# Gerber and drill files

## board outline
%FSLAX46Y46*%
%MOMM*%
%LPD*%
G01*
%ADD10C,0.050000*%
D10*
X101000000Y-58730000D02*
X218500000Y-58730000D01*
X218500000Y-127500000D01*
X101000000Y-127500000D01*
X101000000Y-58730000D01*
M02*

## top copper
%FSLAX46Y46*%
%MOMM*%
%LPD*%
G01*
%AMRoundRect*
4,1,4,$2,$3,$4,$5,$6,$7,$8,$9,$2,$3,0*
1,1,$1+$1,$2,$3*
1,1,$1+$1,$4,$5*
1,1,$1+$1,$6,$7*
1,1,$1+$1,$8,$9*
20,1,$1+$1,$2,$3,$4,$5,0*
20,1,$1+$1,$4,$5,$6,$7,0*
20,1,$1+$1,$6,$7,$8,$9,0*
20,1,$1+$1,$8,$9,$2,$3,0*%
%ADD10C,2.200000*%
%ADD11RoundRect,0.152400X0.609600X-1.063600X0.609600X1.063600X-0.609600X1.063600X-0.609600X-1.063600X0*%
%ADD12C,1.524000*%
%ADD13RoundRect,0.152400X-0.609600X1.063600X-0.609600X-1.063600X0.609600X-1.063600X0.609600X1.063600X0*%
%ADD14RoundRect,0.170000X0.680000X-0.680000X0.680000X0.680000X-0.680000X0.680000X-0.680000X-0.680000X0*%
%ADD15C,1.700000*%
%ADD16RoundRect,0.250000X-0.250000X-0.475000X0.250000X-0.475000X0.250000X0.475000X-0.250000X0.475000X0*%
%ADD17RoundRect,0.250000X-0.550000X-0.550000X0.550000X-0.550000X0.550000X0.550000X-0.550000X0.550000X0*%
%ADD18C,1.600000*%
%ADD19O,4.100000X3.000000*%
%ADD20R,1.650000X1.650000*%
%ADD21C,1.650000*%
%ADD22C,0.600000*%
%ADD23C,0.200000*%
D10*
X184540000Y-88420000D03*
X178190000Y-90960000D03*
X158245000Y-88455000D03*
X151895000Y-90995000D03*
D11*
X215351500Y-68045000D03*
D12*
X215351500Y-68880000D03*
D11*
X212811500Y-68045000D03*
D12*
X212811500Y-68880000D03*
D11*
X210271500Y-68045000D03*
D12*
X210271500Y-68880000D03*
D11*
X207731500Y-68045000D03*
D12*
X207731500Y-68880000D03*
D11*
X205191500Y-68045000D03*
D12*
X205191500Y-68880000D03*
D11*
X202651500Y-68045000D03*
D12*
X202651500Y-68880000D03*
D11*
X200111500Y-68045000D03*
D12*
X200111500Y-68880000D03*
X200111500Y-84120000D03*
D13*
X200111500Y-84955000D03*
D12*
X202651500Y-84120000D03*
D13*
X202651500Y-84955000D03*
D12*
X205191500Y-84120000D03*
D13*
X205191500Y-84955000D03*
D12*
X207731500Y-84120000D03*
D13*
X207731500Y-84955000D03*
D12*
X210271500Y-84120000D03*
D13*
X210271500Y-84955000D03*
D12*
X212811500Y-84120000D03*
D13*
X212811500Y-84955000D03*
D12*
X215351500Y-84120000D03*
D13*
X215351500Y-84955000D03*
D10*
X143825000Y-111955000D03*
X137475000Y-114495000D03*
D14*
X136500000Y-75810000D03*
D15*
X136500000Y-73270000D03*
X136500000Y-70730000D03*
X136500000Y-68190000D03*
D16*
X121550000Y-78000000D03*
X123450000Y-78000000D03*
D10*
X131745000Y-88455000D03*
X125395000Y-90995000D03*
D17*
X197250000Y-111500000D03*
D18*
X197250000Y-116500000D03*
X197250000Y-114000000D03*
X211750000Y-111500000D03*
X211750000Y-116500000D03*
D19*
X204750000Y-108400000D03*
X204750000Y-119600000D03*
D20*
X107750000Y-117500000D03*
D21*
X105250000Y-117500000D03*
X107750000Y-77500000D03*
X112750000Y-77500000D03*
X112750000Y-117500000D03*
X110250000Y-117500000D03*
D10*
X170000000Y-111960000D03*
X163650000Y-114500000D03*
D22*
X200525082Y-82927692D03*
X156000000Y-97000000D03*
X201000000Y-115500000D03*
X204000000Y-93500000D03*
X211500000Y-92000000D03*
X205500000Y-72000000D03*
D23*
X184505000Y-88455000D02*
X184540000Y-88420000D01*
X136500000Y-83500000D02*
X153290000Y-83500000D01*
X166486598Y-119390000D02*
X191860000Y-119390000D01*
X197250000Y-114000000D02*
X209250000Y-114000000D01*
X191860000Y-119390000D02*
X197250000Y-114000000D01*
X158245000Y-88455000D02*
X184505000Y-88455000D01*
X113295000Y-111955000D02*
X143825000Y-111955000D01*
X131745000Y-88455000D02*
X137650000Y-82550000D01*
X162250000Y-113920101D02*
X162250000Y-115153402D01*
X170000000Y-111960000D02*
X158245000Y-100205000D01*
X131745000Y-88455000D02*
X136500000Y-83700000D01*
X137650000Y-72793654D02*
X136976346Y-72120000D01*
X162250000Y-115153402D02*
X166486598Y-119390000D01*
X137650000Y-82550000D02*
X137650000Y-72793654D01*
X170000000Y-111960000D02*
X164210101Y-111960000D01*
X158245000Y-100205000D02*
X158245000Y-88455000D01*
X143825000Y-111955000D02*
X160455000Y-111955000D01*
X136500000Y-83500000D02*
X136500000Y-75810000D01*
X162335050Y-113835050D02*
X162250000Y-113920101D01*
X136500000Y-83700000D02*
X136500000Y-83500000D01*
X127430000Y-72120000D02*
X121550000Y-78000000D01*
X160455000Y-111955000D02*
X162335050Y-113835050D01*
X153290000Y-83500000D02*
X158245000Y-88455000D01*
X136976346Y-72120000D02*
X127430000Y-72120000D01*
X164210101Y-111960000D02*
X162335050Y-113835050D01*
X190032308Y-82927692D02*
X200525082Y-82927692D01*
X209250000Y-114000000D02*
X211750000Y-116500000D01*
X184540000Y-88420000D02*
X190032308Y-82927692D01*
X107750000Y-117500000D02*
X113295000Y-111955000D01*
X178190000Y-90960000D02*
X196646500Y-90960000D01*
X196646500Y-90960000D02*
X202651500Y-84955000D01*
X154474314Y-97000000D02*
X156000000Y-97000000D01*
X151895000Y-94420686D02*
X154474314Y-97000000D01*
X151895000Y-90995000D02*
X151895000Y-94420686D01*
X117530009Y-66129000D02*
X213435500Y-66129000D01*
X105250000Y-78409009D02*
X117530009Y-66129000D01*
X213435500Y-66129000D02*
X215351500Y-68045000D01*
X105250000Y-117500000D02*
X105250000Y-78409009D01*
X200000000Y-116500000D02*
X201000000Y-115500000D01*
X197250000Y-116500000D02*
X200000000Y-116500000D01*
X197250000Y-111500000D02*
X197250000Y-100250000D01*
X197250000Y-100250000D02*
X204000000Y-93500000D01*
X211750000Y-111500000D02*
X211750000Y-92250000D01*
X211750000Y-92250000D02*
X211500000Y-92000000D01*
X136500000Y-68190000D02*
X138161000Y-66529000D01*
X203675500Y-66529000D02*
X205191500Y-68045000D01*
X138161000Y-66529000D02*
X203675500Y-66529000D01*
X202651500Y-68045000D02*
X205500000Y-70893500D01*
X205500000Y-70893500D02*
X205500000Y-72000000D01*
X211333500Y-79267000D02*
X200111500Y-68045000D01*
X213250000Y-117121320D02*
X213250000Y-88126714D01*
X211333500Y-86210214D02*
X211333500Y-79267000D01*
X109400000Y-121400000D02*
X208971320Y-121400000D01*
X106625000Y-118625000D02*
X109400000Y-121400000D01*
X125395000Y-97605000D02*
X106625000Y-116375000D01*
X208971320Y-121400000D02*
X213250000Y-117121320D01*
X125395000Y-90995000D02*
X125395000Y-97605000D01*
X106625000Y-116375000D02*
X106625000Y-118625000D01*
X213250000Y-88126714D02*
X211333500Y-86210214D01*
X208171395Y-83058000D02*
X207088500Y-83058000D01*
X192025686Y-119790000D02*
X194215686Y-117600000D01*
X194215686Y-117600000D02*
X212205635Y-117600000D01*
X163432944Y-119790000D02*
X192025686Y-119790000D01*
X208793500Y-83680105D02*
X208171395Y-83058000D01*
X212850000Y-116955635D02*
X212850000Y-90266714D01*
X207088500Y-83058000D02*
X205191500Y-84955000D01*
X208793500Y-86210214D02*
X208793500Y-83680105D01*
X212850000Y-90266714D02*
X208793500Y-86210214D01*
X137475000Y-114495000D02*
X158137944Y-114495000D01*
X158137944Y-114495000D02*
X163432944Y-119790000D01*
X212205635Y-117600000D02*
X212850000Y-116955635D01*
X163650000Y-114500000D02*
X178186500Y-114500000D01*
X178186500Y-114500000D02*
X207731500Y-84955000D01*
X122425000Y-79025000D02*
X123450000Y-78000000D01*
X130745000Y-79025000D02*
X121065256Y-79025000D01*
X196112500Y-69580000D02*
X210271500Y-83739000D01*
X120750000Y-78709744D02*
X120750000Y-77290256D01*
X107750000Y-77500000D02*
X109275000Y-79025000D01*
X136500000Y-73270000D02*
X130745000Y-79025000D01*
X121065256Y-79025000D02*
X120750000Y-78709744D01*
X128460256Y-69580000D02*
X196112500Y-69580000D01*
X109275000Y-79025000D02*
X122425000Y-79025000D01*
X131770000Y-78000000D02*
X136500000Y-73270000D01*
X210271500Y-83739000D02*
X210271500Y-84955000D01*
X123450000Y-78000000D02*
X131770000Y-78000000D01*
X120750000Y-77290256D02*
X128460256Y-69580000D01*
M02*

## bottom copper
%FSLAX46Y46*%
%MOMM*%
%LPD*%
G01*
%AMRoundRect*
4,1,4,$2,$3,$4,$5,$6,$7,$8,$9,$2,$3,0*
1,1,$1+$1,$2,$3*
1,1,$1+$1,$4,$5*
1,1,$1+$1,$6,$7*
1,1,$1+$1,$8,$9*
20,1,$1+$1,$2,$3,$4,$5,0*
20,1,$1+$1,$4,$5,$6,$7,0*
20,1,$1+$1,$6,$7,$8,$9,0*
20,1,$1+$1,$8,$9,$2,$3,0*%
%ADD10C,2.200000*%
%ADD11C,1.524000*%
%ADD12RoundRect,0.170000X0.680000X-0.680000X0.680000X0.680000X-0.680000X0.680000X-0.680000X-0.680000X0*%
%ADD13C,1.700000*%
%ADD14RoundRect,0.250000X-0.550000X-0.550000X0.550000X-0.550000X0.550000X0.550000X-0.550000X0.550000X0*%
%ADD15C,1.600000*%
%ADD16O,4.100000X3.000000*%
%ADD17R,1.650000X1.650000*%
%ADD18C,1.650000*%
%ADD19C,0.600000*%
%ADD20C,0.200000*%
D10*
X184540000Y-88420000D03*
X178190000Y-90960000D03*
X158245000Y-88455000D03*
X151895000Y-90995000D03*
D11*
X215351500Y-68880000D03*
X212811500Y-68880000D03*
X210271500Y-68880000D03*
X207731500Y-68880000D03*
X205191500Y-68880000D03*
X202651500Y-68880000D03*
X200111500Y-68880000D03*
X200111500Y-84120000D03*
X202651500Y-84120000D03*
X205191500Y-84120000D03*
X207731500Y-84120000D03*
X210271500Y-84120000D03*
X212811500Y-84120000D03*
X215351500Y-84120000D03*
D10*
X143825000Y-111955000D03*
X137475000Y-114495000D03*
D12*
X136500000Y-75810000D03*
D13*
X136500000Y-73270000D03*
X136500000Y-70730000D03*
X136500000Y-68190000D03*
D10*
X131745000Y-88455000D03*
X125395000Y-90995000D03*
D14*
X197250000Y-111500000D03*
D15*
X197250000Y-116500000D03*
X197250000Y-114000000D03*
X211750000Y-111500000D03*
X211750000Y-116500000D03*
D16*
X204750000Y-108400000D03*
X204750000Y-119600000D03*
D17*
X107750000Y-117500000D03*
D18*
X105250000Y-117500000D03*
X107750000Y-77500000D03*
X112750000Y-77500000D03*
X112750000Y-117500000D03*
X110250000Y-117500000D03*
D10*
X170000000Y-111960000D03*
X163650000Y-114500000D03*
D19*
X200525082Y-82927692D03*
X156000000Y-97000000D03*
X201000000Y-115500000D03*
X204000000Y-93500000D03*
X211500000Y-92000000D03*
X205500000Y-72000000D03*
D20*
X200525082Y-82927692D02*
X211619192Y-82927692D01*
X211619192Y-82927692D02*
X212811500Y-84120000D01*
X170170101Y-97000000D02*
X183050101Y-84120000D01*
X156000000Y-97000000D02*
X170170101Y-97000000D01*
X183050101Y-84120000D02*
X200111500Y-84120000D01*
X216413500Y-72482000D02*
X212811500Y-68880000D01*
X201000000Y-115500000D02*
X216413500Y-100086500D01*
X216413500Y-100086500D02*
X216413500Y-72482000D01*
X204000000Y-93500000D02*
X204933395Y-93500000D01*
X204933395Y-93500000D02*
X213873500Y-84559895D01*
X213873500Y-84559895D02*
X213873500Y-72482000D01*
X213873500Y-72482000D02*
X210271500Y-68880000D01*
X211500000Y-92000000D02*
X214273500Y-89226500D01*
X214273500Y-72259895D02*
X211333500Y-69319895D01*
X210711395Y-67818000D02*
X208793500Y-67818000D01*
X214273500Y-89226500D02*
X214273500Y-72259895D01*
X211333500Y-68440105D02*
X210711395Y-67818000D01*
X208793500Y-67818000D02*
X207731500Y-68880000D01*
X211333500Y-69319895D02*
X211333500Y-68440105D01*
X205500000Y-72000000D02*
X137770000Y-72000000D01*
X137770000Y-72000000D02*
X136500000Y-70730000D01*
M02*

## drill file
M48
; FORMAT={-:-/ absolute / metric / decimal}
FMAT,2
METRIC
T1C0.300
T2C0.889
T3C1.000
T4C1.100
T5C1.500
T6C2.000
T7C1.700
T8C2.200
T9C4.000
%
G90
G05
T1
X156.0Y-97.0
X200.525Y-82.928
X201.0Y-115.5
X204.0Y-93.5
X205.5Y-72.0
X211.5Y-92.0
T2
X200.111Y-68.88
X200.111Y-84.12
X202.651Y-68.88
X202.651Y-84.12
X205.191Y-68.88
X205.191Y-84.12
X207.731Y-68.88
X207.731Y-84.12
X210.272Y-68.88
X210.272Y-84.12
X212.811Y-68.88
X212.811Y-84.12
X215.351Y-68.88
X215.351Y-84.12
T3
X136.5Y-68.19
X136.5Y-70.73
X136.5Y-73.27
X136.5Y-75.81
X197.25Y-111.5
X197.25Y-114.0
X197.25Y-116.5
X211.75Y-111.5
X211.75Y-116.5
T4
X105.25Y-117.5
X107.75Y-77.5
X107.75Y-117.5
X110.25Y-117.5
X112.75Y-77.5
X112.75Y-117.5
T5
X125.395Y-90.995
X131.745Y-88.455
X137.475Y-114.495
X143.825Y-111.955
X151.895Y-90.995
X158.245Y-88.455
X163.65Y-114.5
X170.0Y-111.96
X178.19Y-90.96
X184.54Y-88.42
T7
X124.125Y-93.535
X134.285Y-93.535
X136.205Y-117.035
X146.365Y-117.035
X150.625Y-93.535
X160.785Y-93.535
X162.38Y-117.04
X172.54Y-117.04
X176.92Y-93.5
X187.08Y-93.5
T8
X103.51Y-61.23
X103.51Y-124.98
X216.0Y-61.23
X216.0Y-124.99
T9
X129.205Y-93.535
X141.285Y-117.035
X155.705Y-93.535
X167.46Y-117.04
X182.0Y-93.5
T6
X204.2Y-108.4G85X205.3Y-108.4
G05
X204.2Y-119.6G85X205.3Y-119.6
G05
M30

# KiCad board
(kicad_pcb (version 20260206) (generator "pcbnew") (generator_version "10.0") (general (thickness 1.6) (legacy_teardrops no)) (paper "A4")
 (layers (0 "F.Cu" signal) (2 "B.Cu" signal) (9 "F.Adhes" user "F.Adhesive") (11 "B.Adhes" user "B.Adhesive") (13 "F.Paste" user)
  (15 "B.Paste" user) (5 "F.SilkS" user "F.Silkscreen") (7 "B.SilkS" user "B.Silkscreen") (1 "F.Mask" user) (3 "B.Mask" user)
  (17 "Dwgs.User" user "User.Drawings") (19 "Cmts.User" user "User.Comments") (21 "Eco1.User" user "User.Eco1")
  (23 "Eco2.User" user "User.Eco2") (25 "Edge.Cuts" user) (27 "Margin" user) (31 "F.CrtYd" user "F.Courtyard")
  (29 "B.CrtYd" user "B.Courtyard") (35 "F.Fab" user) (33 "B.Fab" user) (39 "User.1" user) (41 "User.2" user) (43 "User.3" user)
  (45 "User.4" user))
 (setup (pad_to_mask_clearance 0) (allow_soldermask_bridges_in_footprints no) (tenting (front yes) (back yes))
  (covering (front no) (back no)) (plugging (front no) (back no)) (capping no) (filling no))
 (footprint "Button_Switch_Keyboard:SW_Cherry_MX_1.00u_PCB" (layer "F.Cu") (at 184.54 88.42)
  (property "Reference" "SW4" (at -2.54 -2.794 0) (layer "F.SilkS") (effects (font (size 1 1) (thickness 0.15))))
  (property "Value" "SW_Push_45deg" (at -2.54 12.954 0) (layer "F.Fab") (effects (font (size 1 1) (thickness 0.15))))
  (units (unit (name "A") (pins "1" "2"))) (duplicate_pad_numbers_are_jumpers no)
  (pad "" np_thru_hole circle (at -7.62 5.08) (size 1.7 1.7) (drill 1.7) (layers "*.Cu" "*.Mask"))
  (pad "" np_thru_hole circle (at -2.54 5.08) (size 4 4) (drill 4) (layers "*.Cu" "*.Mask"))
  (pad "" np_thru_hole circle (at 2.54 5.08) (size 1.7 1.7) (drill 1.7) (layers "*.Cu" "*.Mask"))
  (pad "1" thru_hole circle (at 0 0) (size 2.2 2.2) (drill 1.5) (layers "*.Cu" "*.Mask") (remove_unused_layers no) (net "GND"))
  (pad "2" thru_hole circle (at -6.35 2.54) (size 2.2 2.2) (drill 1.5) (layers "*.Cu" "*.Mask") (remove_unused_layers no) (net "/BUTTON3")))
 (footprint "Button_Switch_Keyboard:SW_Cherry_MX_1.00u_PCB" (layer "F.Cu") (at 158.245 88.455)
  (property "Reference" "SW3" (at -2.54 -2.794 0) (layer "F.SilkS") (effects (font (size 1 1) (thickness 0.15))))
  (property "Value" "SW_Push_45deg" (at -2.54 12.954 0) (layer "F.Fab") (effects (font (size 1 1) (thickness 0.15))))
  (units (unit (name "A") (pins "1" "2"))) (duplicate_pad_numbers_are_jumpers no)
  (pad "" np_thru_hole circle (at -7.62 5.08) (size 1.7 1.7) (drill 1.7) (layers "*.Cu" "*.Mask"))
  (pad "" np_thru_hole circle (at -2.54 5.08) (size 4 4) (drill 4) (layers "*.Cu" "*.Mask"))
  (pad "" np_thru_hole circle (at 2.54 5.08) (size 1.7 1.7) (drill 1.7) (layers "*.Cu" "*.Mask"))
  (pad "1" thru_hole circle (at 0 0) (size 2.2 2.2) (drill 1.5) (layers "*.Cu" "*.Mask") (remove_unused_layers no) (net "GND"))
  (pad "2" thru_hole circle (at -6.35 2.54) (size 2.2 2.2) (drill 1.5) (layers "*.Cu" "*.Mask") (remove_unused_layers no) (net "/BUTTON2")))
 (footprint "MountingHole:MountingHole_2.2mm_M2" (layer "F.Cu") (at 216 124.99)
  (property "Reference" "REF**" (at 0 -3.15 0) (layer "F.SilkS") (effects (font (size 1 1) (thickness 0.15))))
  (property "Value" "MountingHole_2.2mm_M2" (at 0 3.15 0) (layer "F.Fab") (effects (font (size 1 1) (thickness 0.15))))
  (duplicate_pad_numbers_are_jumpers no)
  (pad "" np_thru_hole circle (at 0 0) (size 2.2 2.2) (drill 2.2) (layers "*.Cu" "*.Mask")))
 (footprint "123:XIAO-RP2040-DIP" (layer "F.Cu") (at 207.7315 76.5)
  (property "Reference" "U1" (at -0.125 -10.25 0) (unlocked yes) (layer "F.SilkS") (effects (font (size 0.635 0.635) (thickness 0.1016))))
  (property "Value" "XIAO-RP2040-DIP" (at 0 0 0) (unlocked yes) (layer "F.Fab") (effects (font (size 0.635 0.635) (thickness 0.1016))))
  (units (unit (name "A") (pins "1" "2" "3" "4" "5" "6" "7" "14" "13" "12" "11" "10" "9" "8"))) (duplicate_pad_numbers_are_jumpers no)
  (pad "1" smd roundrect (at 7.62 -8.455 90) (size 2.432 1.524) (layers "F.Cu" "F.Mask") (roundrect_rratio 0.1) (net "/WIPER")
   (thermal_bridge_angle 45))
  (pad "1" thru_hole circle (at 7.62 -7.62 90) (size 1.524 1.524) (drill 0.889) (layers "*.Cu" "*.Mask") (remove_unused_layers no)
   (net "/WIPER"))
  (pad "2" smd roundrect (at 5.08 -8.455 90) (size 2.432 1.524) (layers "F.Cu" "F.Mask") (roundrect_rratio 0.1) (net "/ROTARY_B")
   (thermal_bridge_angle 45))
  (pad "2" thru_hole circle (at 5.08 -7.62 90) (size 1.524 1.524) (drill 0.889) (layers "*.Cu" "*.Mask") (remove_unused_layers no)
   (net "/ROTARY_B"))
  (pad "3" smd roundrect (at 2.54 -8.455 90) (size 2.432 1.524) (layers "F.Cu" "F.Mask") (roundrect_rratio 0.1) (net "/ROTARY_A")
   (thermal_bridge_angle 45))
  (pad "3" thru_hole circle (at 2.54 -7.62 90) (size 1.524 1.524) (drill 0.889) (layers "*.Cu" "*.Mask") (remove_unused_layers no)
   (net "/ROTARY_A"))
  (pad "4" smd roundrect (at 0 -8.455 90) (size 2.432 1.524) (layers "F.Cu" "F.Mask") (roundrect_rratio 0.1) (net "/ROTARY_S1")
   (thermal_bridge_angle 45))
  (pad "4" thru_hole circle (at 0 -7.62 90) (size 1.524 1.524) (drill 0.889) (layers "*.Cu" "*.Mask") (remove_unused_layers no)
   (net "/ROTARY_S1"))
  (pad "5" smd roundrect (at -2.54 -8.455 90) (size 2.432 1.524) (layers "F.Cu" "F.Mask") (roundrect_rratio 0.1) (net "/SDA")
   (thermal_bridge_angle 45))
  (pad "5" thru_hole circle (at -2.54 -7.62 90) (size 1.524 1.524) (drill 0.889) (layers "*.Cu" "*.Mask") (remove_unused_layers no)
   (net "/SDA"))
  (pad "6" smd roundrect (at -5.08 -8.455 90) (size 2.432 1.524) (layers "F.Cu" "F.Mask") (roundrect_rratio 0.1) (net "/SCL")
   (thermal_bridge_angle 45))
  (pad "6" thru_hole circle (at -5.08 -7.62 90) (size 1.524 1.524) (drill 0.889) (layers "*.Cu" "*.Mask") (remove_unused_layers no)
   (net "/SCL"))
  (pad "7" smd roundrect (at -7.62 -8.455 90) (size 2.432 1.524) (layers "F.Cu" "F.Mask") (roundrect_rratio 0.1) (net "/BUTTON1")
   (thermal_bridge_angle 45))
  (pad "7" thru_hole circle (at -7.62 -7.62 90) (size 1.524 1.524) (drill 0.889) (layers "*.Cu" "*.Mask") (remove_unused_layers no)
   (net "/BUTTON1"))
  (pad "8" thru_hole circle (at -7.62 7.62 270) (size 1.524 1.524) (drill 0.889) (layers "*.Cu" "*.Mask") (remove_unused_layers no)
   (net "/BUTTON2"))
  (pad "8" smd roundrect (at -7.62 8.455 270) (size 2.432 1.524) (layers "F.Cu" "F.Mask") (roundrect_rratio 0.1) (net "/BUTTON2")
   (thermal_bridge_angle 45))
  (pad "9" thru_hole circle (at -5.08 7.62 270) (size 1.524 1.524) (drill 0.889) (layers "*.Cu" "*.Mask") (remove_unused_layers no)
   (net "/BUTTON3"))
  (pad "9" smd roundrect (at -5.08 8.455 270) (size 2.432 1.524) (layers "F.Cu" "F.Mask") (roundrect_rratio 0.1) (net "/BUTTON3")
   (thermal_bridge_angle 45))
  (pad "10" thru_hole circle (at -2.54 7.62 270) (size 1.524 1.524) (drill 0.889) (layers "*.Cu" "*.Mask") (remove_unused_layers no)
   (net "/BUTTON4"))
  (pad "10" smd roundrect (at -2.54 8.455 270) (size 2.432 1.524) (layers "F.Cu" "F.Mask") (roundrect_rratio 0.1) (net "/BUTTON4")
   (thermal_bridge_angle 45))
  (pad "11" thru_hole circle (at 0 7.62 270) (size 1.524 1.524) (drill 0.889) (layers "*.Cu" "*.Mask") (remove_unused_layers no)
   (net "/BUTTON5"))
  (pad "11" smd roundrect (at 0 8.455 270) (size 2.432 1.524) (layers "F.Cu" "F.Mask") (roundrect_rratio 0.1) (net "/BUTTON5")
   (thermal_bridge_angle 45))
  (pad "12" thru_hole circle (at 2.54 7.62 270) (size 1.524 1.524) (drill 0.889) (layers "*.Cu" "*.Mask") (remove_unused_layers no)
   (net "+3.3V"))
  (pad "12" smd roundrect (at 2.54 8.455 270) (size 2.432 1.524) (layers "F.Cu" "F.Mask") (roundrect_rratio 0.1) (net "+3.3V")
   (thermal_bridge_angle 45))
  (pad "13" thru_hole circle (at 5.08 7.62 270) (size 1.524 1.524) (drill 0.889) (layers "*.Cu" "*.Mask") (remove_unused_layers no)
   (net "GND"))
  (pad "13" smd roundrect (at 5.08 8.455 270) (size 2.432 1.524) (layers "F.Cu" "F.Mask") (roundrect_rratio 0.1) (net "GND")
   (thermal_bridge_angle 45))
  (pad "14" thru_hole circle (at 7.62 7.62 270) (size 1.524 1.524) (drill 0.889) (layers "*.Cu" "*.Mask") (remove_unused_layers no)
   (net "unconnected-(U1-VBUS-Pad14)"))
  (pad "14" smd roundrect (at 7.62 8.455 270) (size 2.432 1.524) (layers "F.Cu" "F.Mask") (roundrect_rratio 0.1)
   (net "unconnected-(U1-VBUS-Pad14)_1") (thermal_bridge_angle 45)))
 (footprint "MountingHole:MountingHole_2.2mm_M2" (layer "F.Cu") (at 103.51 124.98)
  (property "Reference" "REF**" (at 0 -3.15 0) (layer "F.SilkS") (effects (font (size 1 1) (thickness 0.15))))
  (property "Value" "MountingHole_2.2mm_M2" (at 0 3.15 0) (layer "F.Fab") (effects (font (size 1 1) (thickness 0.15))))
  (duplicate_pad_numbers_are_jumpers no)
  (pad "" np_thru_hole circle (at 0 0) (size 2.2 2.2) (drill 2.2) (layers "*.Cu" "*.Mask")))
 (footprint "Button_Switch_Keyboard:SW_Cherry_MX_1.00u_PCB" (layer "F.Cu") (at 143.825 111.955)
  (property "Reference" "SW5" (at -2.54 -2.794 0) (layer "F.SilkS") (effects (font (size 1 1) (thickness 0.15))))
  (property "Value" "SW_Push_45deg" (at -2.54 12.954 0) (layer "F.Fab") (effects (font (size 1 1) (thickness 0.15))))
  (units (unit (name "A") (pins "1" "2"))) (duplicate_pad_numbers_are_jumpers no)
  (pad "" np_thru_hole circle (at -7.62 5.08) (size 1.7 1.7) (drill 1.7) (layers "*.Cu" "*.Mask"))
  (pad "" np_thru_hole circle (at -2.54 5.08) (size 4 4) (drill 4) (layers "*.Cu" "*.Mask"))
  (pad "" np_thru_hole circle (at 2.54 5.08) (size 1.7 1.7) (drill 1.7) (layers "*.Cu" "*.Mask"))
  (pad "1" thru_hole circle (at 0 0) (size 2.2 2.2) (drill 1.5) (layers "*.Cu" "*.Mask") (remove_unused_layers no) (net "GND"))
  (pad "2" thru_hole circle (at -6.35 2.54) (size 2.2 2.2) (drill 1.5) (layers "*.Cu" "*.Mask") (remove_unused_layers no) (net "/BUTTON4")))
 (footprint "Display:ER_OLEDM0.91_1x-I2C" (layer "F.Cu") (at 136.5 75.81 90)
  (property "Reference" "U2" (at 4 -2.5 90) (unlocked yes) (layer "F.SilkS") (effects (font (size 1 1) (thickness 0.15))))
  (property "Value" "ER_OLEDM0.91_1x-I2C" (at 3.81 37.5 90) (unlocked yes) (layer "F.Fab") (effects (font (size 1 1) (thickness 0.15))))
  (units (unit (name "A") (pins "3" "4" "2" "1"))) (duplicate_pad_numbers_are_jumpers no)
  (pad "1" thru_hole roundrect (at 0 0 90) (size 1.7 1.7) (drill 1) (layers "*.Cu" "*.Mask") (remove_unused_layers no)
   (roundrect_rratio 0.1) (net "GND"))
  (pad "2" thru_hole circle (at 2.54 0 90) (size 1.7 1.7) (drill 1) (layers "*.Cu" "*.Mask") (remove_unused_layers no) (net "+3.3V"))
  (pad "3" thru_hole circle (at 5.08 0 90) (size 1.7 1.7) (drill 1) (layers "*.Cu" "*.Mask") (remove_unused_layers no) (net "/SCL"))
  (pad "4" thru_hole circle (at 7.62 0 90) (size 1.7 1.7) (drill 1) (layers "*.Cu" "*.Mask") (remove_unused_layers no) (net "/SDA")))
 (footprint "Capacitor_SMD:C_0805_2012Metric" (layer "F.Cu") (at 122.5 78)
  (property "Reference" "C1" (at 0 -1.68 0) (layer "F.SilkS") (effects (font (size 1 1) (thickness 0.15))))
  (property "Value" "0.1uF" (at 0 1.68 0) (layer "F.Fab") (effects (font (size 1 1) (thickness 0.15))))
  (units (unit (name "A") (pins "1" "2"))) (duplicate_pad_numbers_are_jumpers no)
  (pad "1" smd roundrect (at -0.95 0) (size 1 1.45) (layers "F.Cu" "F.Mask" "F.Paste") (roundrect_rratio 0.25) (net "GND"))
  (pad "2" smd roundrect (at 0.95 0) (size 1 1.45) (layers "F.Cu" "F.Mask" "F.Paste") (roundrect_rratio 0.25) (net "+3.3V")))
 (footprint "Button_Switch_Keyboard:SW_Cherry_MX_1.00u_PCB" (layer "F.Cu") (at 131.745 88.455)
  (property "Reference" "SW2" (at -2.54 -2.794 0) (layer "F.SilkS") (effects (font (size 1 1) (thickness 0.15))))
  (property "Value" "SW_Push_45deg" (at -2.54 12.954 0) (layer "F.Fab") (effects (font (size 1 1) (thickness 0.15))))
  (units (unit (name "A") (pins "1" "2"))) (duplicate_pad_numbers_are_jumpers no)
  (pad "" np_thru_hole circle (at -7.62 5.08) (size 1.7 1.7) (drill 1.7) (layers "*.Cu" "*.Mask"))
  (pad "" np_thru_hole circle (at -2.54 5.08) (size 4 4) (drill 4) (layers "*.Cu" "*.Mask"))
  (pad "" np_thru_hole circle (at 2.54 5.08) (size 1.7 1.7) (drill 1.7) (layers "*.Cu" "*.Mask"))
  (pad "1" thru_hole circle (at 0 0) (size 2.2 2.2) (drill 1.5) (layers "*.Cu" "*.Mask") (remove_unused_layers no) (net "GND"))
  (pad "2" thru_hole circle (at -6.35 2.54) (size 2.2 2.2) (drill 1.5) (layers "*.Cu" "*.Mask") (remove_unused_layers no) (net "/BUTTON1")))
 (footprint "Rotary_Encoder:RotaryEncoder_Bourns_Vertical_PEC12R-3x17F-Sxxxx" (layer "F.Cu") (at 197.25 111.5)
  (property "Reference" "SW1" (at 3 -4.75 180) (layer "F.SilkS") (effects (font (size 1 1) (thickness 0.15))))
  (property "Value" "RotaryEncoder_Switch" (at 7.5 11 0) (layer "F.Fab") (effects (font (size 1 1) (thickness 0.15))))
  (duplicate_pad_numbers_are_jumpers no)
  (pad "A" thru_hole roundrect (at 0 0) (size 1.6 1.6) (drill 1) (layers "*.Cu" "*.Mask") (remove_unused_layers no)
   (roundrect_rratio 0.15625) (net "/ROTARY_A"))
  (pad "B" thru_hole circle (at 0 5) (size 1.6 1.6) (drill 1) (layers "*.Cu" "*.Mask") (remove_unused_layers no) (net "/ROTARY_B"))
  (pad "C" thru_hole circle (at 0 2.5) (size 1.6 1.6) (drill 1) (layers "*.Cu" "*.Mask") (remove_unused_layers no) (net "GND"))
  (pad "S1" thru_hole circle (at 14.5 0) (size 1.6 1.6) (drill 1) (layers "*.Cu" "*.Mask") (remove_unused_layers no) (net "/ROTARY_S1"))
  (pad "S2" thru_hole circle (at 14.5 5) (size 1.6 1.6) (drill 1) (layers "*.Cu" "*.Mask") (remove_unused_layers no) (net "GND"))
  (pad "SH" thru_hole oval (at 7.5 -3.1) (size 4.1 3) (drill oval 3.1 2) (layers "*.Cu" "*.Mask") (remove_unused_layers no))
  (pad "SH" thru_hole oval (at 7.5 8.1) (size 4.1 3) (drill oval 3.1 2) (layers "*.Cu" "*.Mask") (remove_unused_layers no)))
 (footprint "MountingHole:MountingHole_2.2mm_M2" (layer "F.Cu") (at 216 61.23)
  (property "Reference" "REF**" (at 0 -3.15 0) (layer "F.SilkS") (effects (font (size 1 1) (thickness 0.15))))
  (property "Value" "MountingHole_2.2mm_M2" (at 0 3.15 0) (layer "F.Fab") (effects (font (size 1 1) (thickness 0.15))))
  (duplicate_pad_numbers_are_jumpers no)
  (pad "" np_thru_hole circle (at 0 0) (size 2.2 2.2) (drill 2.2) (layers "*.Cu" "*.Mask")))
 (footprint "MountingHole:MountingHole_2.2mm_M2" (layer "F.Cu") (at 103.51 61.23)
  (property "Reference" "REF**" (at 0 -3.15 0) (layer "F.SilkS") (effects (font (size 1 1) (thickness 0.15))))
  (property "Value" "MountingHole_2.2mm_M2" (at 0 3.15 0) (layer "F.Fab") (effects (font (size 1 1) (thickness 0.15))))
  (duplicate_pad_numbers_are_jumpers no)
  (pad "" np_thru_hole circle (at 0 0) (size 2.2 2.2) (drill 2.2) (layers "*.Cu" "*.Mask")))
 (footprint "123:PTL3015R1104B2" (layer "F.Cu") (at 107.75 117.5 90)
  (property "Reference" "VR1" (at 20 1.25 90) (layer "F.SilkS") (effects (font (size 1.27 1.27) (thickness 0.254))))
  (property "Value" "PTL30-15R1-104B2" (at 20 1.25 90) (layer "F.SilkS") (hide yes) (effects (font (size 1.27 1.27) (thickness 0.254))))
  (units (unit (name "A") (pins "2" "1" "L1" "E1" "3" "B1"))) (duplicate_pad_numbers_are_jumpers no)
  (pad "1" thru_hole rect (at 0 0 90) (size 1.65 1.65) (drill 1.1) (layers "*.Cu" "*.Mask") (remove_unused_layers no) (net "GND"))
  (pad "2" thru_hole circle (at 0 -2.5 90) (size 1.65 1.65) (drill 1.1) (layers "*.Cu" "*.Mask") (remove_unused_layers no) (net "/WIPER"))
  (pad "3" thru_hole circle (at 40 0 90) (size 1.65 1.65) (drill 1.1) (layers "*.Cu" "*.Mask") (remove_unused_layers no) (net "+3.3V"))
  (pad "B1" thru_hole circle (at 40 5 90) (size 1.65 1.65) (drill 1.1) (layers "*.Cu" "*.Mask") (remove_unused_layers no)
   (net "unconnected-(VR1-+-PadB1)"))
  (pad "E1" thru_hole circle (at 0 5 90) (size 1.65 1.65) (drill 1.1) (layers "*.Cu" "*.Mask") (remove_unused_layers no)
   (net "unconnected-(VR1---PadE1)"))
  (pad "L1" thru_hole circle (at 0 2.5 90) (size 1.65 1.65) (drill 1.1) (layers "*.Cu" "*.Mask") (remove_unused_layers no)
   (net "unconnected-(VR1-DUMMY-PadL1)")))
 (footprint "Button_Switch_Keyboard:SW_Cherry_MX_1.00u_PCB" (layer "F.Cu") (at 170 111.96)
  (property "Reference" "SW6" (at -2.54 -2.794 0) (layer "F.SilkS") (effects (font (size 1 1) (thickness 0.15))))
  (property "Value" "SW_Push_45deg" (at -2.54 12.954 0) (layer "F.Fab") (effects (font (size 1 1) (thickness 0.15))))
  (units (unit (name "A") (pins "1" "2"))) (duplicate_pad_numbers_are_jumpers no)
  (pad "" np_thru_hole circle (at -7.62 5.08) (size 1.7 1.7) (drill 1.7) (layers "*.Cu" "*.Mask"))
  (pad "" np_thru_hole circle (at -2.54 5.08) (size 4 4) (drill 4) (layers "*.Cu" "*.Mask"))
  (pad "" np_thru_hole circle (at 2.54 5.08) (size 1.7 1.7) (drill 1.7) (layers "*.Cu" "*.Mask"))
  (pad "1" thru_hole circle (at 0 0) (size 2.2 2.2) (drill 1.5) (layers "*.Cu" "*.Mask") (remove_unused_layers no) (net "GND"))
  (pad "2" thru_hole circle (at -6.35 2.54) (size 2.2 2.2) (drill 1.5) (layers "*.Cu" "*.Mask") (remove_unused_layers no) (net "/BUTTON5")))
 (gr_rect (start 101 58.73) (end 218.5 127.5) (stroke (width 0.05) (type default)) (fill no) (layer "Edge.Cuts"))
 (segment (start 184.505 88.455) (end 184.54 88.42) (width 0.2) (layer "F.Cu") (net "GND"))
 (segment (start 136.5 83.5) (end 153.29 83.5) (width 0.2) (layer "F.Cu") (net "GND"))
 (segment (start 166.486598 119.39) (end 191.86 119.39) (width 0.2) (layer "F.Cu") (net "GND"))
 (segment (start 197.25 114) (end 209.25 114) (width 0.2) (layer "F.Cu") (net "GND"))
 (segment (start 191.86 119.39) (end 197.25 114) (width 0.2) (layer "F.Cu") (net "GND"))
 (segment (start 158.245 88.455) (end 184.505 88.455) (width 0.2) (layer "F.Cu") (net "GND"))
 (segment (start 113.295 111.955) (end 143.825 111.955) (width 0.2) (layer "F.Cu") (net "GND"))
 (segment (start 131.745 88.455) (end 137.65 82.55) (width 0.2) (layer "F.Cu") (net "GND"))
 (segment (start 162.25 113.920101) (end 162.25 115.153402) (width 0.2) (layer "F.Cu") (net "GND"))
 (segment (start 170 111.96) (end 158.245 100.205) (width 0.2) (layer "F.Cu") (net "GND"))
 (segment (start 131.745 88.455) (end 136.5 83.7) (width 0.2) (layer "F.Cu") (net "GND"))
 (segment (start 137.65 72.793654) (end 136.976346 72.12) (width 0.2) (layer "F.Cu") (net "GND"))
 (segment (start 162.25 115.153402) (end 166.486598 119.39) (width 0.2) (layer "F.Cu") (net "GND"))
 (segment (start 137.65 82.55) (end 137.65 72.793654) (width 0.2) (layer "F.Cu") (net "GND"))
 (segment (start 170 111.96) (end 164.210101 111.96) (width 0.2) (layer "F.Cu") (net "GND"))
 (segment (start 158.245 100.205) (end 158.245 88.455) (width 0.2) (layer "F.Cu") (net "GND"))
 (segment (start 143.825 111.955) (end 160.455 111.955) (width 0.2) (layer "F.Cu") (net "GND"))
 (segment (start 136.5 83.5) (end 136.5 75.81) (width 0.2) (layer "F.Cu") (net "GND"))
 (segment (start 162.33505 113.83505) (end 162.25 113.920101) (width 0.2) (layer "F.Cu") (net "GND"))
 (segment (start 136.5 83.7) (end 136.5 83.5) (width 0.2) (layer "F.Cu") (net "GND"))
 (segment (start 127.43 72.12) (end 121.55 78) (width 0.2) (layer "F.Cu") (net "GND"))
 (segment (start 160.455 111.955) (end 162.33505 113.83505) (width 0.2) (layer "F.Cu") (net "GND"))
 (segment (start 153.29 83.5) (end 158.245 88.455) (width 0.2) (layer "F.Cu") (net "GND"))
 (segment (start 136.976346 72.12) (end 127.43 72.12) (width 0.2) (layer "F.Cu") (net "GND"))
 (segment (start 164.210101 111.96) (end 162.33505 113.83505) (width 0.2) (layer "F.Cu") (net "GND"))
 (segment (start 190.032308 82.927692) (end 200.525082 82.927692) (width 0.2) (layer "F.Cu") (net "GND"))
 (segment (start 209.25 114) (end 211.75 116.5) (width 0.2) (layer "F.Cu") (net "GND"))
 (segment (start 184.54 88.42) (end 190.032308 82.927692) (width 0.2) (layer "F.Cu") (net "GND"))
 (segment (start 107.75 117.5) (end 113.295 111.955) (width 0.2) (layer "F.Cu") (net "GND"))
 (via (at 200.525082 82.927692) (size 0.6) (drill 0.3) (layers "F.Cu" "B.Cu") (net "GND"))
 (segment (start 200.525082 82.927692) (end 211.619192 82.927692) (width 0.2) (layer "B.Cu") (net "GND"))
 (segment (start 211.619192 82.927692) (end 212.8115 84.12) (width 0.2) (layer "B.Cu") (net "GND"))
 (segment (start 178.19 90.96) (end 196.6465 90.96) (width 0.2) (layer "F.Cu") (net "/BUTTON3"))
 (segment (start 196.6465 90.96) (end 202.6515 84.955) (width 0.2) (layer "F.Cu") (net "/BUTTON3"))
 (segment (start 154.474314 97) (end 156 97) (width 0.2) (layer "F.Cu") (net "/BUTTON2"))
 (segment (start 151.895 94.420686) (end 154.474314 97) (width 0.2) (layer "F.Cu") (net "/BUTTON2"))
 (segment (start 151.895 90.995) (end 151.895 94.420686) (width 0.2) (layer "F.Cu") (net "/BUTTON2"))
 (via (at 156 97) (size 0.6) (drill 0.3) (layers "F.Cu" "B.Cu") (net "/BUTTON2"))
 (segment (start 170.170101 97) (end 183.050101 84.12) (width 0.2) (layer "B.Cu") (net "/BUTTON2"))
 (segment (start 156 97) (end 170.170101 97) (width 0.2) (layer "B.Cu") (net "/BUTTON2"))
 (segment (start 183.050101 84.12) (end 200.1115 84.12) (width 0.2) (layer "B.Cu") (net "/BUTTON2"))
 (segment (start 117.530009 66.129) (end 213.4355 66.129) (width 0.2) (layer "F.Cu") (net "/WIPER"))
 (segment (start 105.25 78.409009) (end 117.530009 66.129) (width 0.2) (layer "F.Cu") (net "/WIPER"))
 (segment (start 213.4355 66.129) (end 215.3515 68.045) (width 0.2) (layer "F.Cu") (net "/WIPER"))
 (segment (start 105.25 117.5) (end 105.25 78.409009) (width 0.2) (layer "F.Cu") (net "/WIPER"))
 (segment (start 200 116.5) (end 201 115.5) (width 0.2) (layer "F.Cu") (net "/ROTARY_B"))
 (segment (start 197.25 116.5) (end 200 116.5) (width 0.2) (layer "F.Cu") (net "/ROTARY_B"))
 (via (at 201 115.5) (size 0.6) (drill 0.3) (layers "F.Cu" "B.Cu") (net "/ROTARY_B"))
 (segment (start 216.4135 72.482) (end 212.8115 68.88) (width 0.2) (layer "B.Cu") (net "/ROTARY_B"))
 (segment (start 201 115.5) (end 216.4135 100.0865) (width 0.2) (layer "B.Cu") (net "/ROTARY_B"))
 (segment (start 216.4135 100.0865) (end 216.4135 72.482) (width 0.2) (layer "B.Cu") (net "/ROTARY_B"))
 (segment (start 197.25 111.5) (end 197.25 100.25) (width 0.2) (layer "F.Cu") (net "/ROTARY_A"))
 (segment (start 197.25 100.25) (end 204 93.5) (width 0.2) (layer "F.Cu") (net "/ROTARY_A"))
 (via (at 204 93.5) (size 0.6) (drill 0.3) (layers "F.Cu" "B.Cu") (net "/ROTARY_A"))
 (segment (start 204 93.5) (end 204.933395 93.5) (width 0.2) (layer "B.Cu") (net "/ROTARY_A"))
 (segment (start 204.933395 93.5) (end 213.8735 84.559895) (width 0.2) (layer "B.Cu") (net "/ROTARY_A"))
 (segment (start 213.8735 84.559895) (end 213.8735 72.482) (width 0.2) (layer "B.Cu") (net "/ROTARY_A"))
 (segment (start 213.8735 72.482) (end 210.2715 68.88) (width 0.2) (layer "B.Cu") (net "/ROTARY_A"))
 (segment (start 211.75 111.5) (end 211.75 92.25) (width 0.2) (layer "F.Cu") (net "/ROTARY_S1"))
 (segment (start 211.75 92.25) (end 211.5 92) (width 0.2) (layer "F.Cu") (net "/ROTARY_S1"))
 (via (at 211.5 92) (size 0.6) (drill 0.3) (layers "F.Cu" "B.Cu") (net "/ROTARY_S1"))
 (segment (start 211.5 92) (end 214.2735 89.2265) (width 0.2) (layer "B.Cu") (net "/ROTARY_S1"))
 (segment (start 214.2735 72.259895) (end 211.3335 69.319895) (width 0.2) (layer "B.Cu") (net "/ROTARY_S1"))
 (segment (start 210.711395 67.818) (end 208.7935 67.818) (width 0.2) (layer "B.Cu") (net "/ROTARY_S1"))
 (segment (start 214.2735 89.2265) (end 214.2735 72.259895) (width 0.2) (layer "B.Cu") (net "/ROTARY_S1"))
 (segment (start 211.3335 68.440105) (end 210.711395 67.818) (width 0.2) (layer "B.Cu") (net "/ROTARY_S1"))
 (segment (start 208.7935 67.818) (end 207.7315 68.88) (width 0.2) (layer "B.Cu") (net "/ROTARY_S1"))
 (segment (start 211.3335 69.319895) (end 211.3335 68.440105) (width 0.2) (layer "B.Cu") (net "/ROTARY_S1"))
 (segment (start 136.5 68.19) (end 138.161 66.529) (width 0.2) (layer "F.Cu") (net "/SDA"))
 (segment (start 203.6755 66.529) (end 205.1915 68.045) (width 0.2) (layer "F.Cu") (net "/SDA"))
 (segment (start 138.161 66.529) (end 203.6755 66.529) (width 0.2) (layer "F.Cu") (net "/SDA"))
 (segment (start 202.6515 68.045) (end 205.5 70.8935) (width 0.2) (layer "F.Cu") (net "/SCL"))
 (segment (start 205.5 70.8935) (end 205.5 72) (width 0.2) (layer "F.Cu") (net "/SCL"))
 (via (at 205.5 72) (size 0.6) (drill 0.3) (layers "F.Cu" "B.Cu") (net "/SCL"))
 (segment (start 205.5 72) (end 137.77 72) (width 0.2) (layer "B.Cu") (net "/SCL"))
 (segment (start 137.77 72) (end 136.5 70.73) (width 0.2) (layer "B.Cu") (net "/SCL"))
 (segment (start 211.3335 79.267) (end 200.1115 68.045) (width 0.2) (layer "F.Cu") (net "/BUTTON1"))
 (segment (start 213.25 117.12132) (end 213.25 88.126714) (width 0.2) (layer "F.Cu") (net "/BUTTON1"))
 (segment (start 211.3335 86.210214) (end 211.3335 79.267) (width 0.2) (layer "F.Cu") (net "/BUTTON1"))
 (segment (start 109.4 121.4) (end 208.97132 121.4) (width 0.2) (layer "F.Cu") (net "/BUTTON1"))
 (segment (start 106.625 118.625) (end 109.4 121.4) (width 0.2) (layer "F.Cu") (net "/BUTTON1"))
 (segment (start 125.395 97.605) (end 106.625 116.375) (width 0.2) (layer "F.Cu") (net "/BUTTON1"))
 (segment (start 208.97132 121.4) (end 213.25 117.12132) (width 0.2) (layer "F.Cu") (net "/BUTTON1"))
 (segment (start 125.395 90.995) (end 125.395 97.605) (width 0.2) (layer "F.Cu") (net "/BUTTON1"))
 (segment (start 106.625 116.375) (end 106.625 118.625) (width 0.2) (layer "F.Cu") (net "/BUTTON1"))
 (segment (start 213.25 88.126714) (end 211.3335 86.210214) (width 0.2) (layer "F.Cu") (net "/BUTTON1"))
 (segment (start 208.171395 83.058) (end 207.0885 83.058) (width 0.2) (layer "F.Cu") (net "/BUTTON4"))
 (segment (start 192.025686 119.79) (end 194.215686 117.6) (width 0.2) (layer "F.Cu") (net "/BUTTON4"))
 (segment (start 194.215686 117.6) (end 212.205635 117.6) (width 0.2) (layer "F.Cu") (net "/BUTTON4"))
 (segment (start 163.432944 119.79) (end 192.025686 119.79) (width 0.2) (layer "F.Cu") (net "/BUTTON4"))
 (segment (start 208.7935 83.680105) (end 208.171395 83.058) (width 0.2) (layer "F.Cu") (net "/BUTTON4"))
 (segment (start 212.85 116.955635) (end 212.85 90.266714) (width 0.2) (layer "F.Cu") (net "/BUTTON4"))
 (segment (start 207.0885 83.058) (end 205.1915 84.955) (width 0.2) (layer "F.Cu") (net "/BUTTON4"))
 (segment (start 208.7935 86.210214) (end 208.7935 83.680105) (width 0.2) (layer "F.Cu") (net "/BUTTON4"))
 (segment (start 212.85 90.266714) (end 208.7935 86.210214) (width 0.2) (layer "F.Cu") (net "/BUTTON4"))
 (segment (start 137.475 114.495) (end 158.137944 114.495) (width 0.2) (layer "F.Cu") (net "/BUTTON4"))
 (segment (start 158.137944 114.495) (end 163.432944 119.79) (width 0.2) (layer "F.Cu") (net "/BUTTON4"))
 (segment (start 212.205635 117.6) (end 212.85 116.955635) (width 0.2) (layer "F.Cu") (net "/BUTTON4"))
 (segment (start 163.65 114.5) (end 178.1865 114.5) (width 0.2) (layer "F.Cu") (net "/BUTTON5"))
 (segment (start 178.1865 114.5) (end 207.7315 84.955) (width 0.2) (layer "F.Cu") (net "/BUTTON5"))
 (segment (start 122.425 79.025) (end 123.45 78) (width 0.2) (layer "F.Cu") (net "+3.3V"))
 (segment (start 130.745 79.025) (end 121.065256 79.025) (width 0.2) (layer "F.Cu") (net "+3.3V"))
 (segment (start 196.1125 69.58) (end 210.2715 83.739) (width 0.2) (layer "F.Cu") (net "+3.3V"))
 (segment (start 120.75 78.709744) (end 120.75 77.290256) (width 0.2) (layer "F.Cu") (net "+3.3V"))
 (segment (start 107.75 77.5) (end 109.275 79.025) (width 0.2) (layer "F.Cu") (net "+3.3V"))
 (segment (start 136.5 73.27) (end 130.745 79.025) (width 0.2) (layer "F.Cu") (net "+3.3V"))
 (segment (start 121.065256 79.025) (end 120.75 78.709744) (width 0.2) (layer "F.Cu") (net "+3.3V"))
 (segment (start 128.460256 69.58) (end 196.1125 69.58) (width 0.2) (layer "F.Cu") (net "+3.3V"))
 (segment (start 109.275 79.025) (end 122.425 79.025) (width 0.2) (layer "F.Cu") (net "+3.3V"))
 (segment (start 131.77 78) (end 136.5 73.27) (width 0.2) (layer "F.Cu") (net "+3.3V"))
 (segment (start 210.2715 83.739) (end 210.2715 84.955) (width 0.2) (layer "F.Cu") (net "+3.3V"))
 (segment (start 123.45 78) (end 131.77 78) (width 0.2) (layer "F.Cu") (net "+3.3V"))
 (segment (start 120.75 77.290256) (end 128.460256 69.58) (width 0.2) (layer "F.Cu") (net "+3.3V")))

